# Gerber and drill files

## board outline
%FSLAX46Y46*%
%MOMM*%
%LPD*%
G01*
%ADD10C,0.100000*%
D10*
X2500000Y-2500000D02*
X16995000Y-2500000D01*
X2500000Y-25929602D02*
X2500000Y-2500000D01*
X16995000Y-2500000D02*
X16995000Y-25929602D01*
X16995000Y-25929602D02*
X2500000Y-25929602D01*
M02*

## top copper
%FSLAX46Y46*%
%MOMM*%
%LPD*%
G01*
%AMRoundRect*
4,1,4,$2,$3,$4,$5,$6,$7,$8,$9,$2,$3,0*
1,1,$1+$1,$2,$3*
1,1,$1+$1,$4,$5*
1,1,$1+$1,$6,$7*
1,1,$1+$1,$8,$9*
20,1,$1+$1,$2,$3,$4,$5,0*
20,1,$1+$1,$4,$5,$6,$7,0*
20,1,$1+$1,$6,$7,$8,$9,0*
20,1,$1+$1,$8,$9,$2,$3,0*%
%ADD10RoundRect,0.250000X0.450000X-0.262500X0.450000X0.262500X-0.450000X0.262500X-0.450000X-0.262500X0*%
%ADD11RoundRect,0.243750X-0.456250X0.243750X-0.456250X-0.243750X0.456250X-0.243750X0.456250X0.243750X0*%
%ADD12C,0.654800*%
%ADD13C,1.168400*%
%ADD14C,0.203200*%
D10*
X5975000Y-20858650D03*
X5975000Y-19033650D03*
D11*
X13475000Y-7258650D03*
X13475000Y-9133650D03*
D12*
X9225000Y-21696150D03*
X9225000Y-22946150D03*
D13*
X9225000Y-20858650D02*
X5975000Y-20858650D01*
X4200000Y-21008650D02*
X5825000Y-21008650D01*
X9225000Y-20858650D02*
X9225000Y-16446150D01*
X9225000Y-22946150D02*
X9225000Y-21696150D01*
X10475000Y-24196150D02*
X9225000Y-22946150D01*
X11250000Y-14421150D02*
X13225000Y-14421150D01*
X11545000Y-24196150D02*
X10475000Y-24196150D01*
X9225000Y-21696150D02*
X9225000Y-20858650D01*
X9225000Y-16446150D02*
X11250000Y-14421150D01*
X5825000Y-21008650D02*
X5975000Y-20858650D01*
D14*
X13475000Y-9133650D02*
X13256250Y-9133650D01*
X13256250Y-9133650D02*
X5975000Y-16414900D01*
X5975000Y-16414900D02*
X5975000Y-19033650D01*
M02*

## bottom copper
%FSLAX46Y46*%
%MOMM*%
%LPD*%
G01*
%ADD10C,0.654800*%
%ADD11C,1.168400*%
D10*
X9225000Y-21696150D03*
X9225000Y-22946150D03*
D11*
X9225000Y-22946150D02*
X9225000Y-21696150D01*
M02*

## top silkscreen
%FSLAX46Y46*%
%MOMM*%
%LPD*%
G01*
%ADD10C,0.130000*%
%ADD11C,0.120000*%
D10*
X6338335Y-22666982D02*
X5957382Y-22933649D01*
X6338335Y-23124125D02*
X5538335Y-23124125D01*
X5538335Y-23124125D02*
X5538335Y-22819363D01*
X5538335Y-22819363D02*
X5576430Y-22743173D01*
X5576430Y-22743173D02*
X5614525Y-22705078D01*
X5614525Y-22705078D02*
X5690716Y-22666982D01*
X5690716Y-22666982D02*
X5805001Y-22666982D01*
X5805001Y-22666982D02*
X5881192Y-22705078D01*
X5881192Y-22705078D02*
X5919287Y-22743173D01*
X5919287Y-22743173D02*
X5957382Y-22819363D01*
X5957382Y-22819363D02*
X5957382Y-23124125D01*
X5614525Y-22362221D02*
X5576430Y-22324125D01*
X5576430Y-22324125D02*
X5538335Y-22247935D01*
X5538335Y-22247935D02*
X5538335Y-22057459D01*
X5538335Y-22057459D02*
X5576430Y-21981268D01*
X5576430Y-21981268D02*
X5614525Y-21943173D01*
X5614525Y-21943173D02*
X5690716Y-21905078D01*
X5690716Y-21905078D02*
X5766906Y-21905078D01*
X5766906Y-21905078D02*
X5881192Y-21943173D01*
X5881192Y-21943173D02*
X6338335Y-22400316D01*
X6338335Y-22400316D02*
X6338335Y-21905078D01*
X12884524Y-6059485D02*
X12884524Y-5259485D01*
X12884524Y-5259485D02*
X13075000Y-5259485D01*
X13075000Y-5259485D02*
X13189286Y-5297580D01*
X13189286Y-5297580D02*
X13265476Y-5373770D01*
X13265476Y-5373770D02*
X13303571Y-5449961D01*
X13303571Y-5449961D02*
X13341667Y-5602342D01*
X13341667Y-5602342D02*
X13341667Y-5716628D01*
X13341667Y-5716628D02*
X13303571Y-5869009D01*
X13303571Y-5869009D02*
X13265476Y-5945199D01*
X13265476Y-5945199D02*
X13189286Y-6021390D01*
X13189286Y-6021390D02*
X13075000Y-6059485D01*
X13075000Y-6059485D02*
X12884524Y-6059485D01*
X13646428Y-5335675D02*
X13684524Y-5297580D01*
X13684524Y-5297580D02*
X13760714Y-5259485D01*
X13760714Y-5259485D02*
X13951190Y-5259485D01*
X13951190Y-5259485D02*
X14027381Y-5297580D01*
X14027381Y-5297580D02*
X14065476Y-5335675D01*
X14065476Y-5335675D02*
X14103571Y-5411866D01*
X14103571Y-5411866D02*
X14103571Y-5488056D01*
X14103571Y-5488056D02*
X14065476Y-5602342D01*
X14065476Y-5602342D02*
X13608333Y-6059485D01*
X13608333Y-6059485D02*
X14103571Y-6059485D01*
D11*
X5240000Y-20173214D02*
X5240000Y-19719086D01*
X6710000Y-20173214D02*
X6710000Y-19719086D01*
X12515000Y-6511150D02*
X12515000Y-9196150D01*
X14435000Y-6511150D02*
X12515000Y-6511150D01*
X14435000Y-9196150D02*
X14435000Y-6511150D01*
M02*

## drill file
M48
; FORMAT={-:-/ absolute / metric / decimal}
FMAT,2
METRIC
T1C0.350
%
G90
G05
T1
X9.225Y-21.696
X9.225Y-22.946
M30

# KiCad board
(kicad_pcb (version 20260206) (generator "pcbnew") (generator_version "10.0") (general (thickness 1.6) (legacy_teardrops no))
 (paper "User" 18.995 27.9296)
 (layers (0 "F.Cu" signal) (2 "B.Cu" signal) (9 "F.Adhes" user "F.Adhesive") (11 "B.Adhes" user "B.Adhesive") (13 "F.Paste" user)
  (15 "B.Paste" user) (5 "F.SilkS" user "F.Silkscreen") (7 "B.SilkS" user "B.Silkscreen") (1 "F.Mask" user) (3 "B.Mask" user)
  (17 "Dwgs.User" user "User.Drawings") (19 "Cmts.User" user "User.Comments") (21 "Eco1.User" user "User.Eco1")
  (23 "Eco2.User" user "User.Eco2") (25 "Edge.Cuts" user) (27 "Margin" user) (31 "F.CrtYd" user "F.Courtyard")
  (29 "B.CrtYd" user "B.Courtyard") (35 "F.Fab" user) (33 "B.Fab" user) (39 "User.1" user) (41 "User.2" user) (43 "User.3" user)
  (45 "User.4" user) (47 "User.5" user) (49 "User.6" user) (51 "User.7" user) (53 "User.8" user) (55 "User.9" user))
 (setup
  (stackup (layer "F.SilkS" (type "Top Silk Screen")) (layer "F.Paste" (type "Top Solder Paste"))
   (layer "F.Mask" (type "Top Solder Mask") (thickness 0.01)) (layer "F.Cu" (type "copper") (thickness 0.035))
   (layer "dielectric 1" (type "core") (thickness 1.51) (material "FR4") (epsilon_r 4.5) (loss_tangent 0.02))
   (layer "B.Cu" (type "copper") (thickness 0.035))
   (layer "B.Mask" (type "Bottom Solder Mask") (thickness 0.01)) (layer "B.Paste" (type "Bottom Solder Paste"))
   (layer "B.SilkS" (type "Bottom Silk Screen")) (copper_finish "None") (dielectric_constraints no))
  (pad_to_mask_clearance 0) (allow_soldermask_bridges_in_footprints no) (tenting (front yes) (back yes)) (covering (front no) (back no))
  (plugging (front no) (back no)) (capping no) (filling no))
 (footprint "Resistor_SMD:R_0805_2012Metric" (layer "F.Cu") (at 5.975 19.94615 90)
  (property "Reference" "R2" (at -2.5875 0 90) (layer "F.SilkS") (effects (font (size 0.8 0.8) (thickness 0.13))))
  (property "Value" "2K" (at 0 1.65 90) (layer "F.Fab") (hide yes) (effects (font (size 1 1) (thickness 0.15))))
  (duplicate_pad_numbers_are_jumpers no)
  (fp_line (start -0.227064 -0.735) (end 0.227064 -0.735) (stroke (width 0.12) (type solid)) (layer "F.SilkS"))
  (fp_line (start -0.227064 0.735) (end 0.227064 0.735) (stroke (width 0.12) (type solid)) (layer "F.SilkS"))
  (pad "1" smd roundrect (at -0.9125 0 90) (size 1.025 1.4) (layers "F.Cu" "F.Mask" "F.Paste") (roundrect_rratio 0.243902439) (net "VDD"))
  (pad "2" smd roundrect (at 0.9125 0 90) (size 1.025 1.4) (layers "F.Cu" "F.Mask" "F.Paste") (roundrect_rratio 0.243902439)
   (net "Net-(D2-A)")))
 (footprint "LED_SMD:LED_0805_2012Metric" (layer "F.Cu") (at 13.475 8.19615 -90)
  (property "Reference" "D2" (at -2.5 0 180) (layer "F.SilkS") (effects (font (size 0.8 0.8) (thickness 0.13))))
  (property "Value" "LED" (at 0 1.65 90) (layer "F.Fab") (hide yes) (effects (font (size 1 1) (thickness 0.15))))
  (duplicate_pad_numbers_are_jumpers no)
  (fp_line (start -1.685 0.96) (end 1 0.96) (stroke (width 0.12) (type solid)) (layer "F.SilkS"))
  (fp_line (start -1.685 -0.96) (end -1.685 0.96) (stroke (width 0.12) (type solid)) (layer "F.SilkS"))
  (fp_line (start 1 -0.96) (end -1.685 -0.96) (stroke (width 0.12) (type solid)) (layer "F.SilkS"))
  (pad "1" smd roundrect (at -0.9375 0 270) (size 0.975 1.4) (layers "F.Cu" "F.Mask" "F.Paste") (roundrect_rratio 0.25) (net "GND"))
  (pad "2" smd roundrect (at 0.9375 0 270) (size 0.975 1.4) (layers "F.Cu" "F.Mask" "F.Paste") (roundrect_rratio 0.25) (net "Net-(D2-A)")))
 (gr_line (start 2.5 2.5) (end 16.995 2.5) (stroke (width 0.1) (type default)) (layer "Edge.Cuts"))
 (gr_line (start 2.5 25.929602) (end 2.5 2.5) (stroke (width 0.1) (type default)) (layer "Edge.Cuts"))
 (gr_line (start 16.995 2.5) (end 16.995 25.929602) (stroke (width 0.1) (type default)) (layer "Edge.Cuts"))
 (gr_line (start 16.995 25.929602) (end 2.5 25.929602) (stroke (width 0.1) (type default)) (layer "Edge.Cuts"))
 (segment (start 9.225 20.85865) (end 5.975 20.85865) (width 1.1684) (layer "F.Cu") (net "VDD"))
 (segment (start 4.2 21.00865) (end 5.825 21.00865) (width 1.1684) (layer "F.Cu") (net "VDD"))
 (segment (start 9.225 20.85865) (end 9.225 16.44615) (width 1.1684) (layer "F.Cu") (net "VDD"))
 (segment (start 9.225 22.94615) (end 9.225 21.69615) (width 1.1684) (layer "F.Cu") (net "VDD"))
 (segment (start 10.475 24.19615) (end 9.225 22.94615) (width 1.1684) (layer "F.Cu") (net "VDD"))
 (segment (start 11.25 14.42115) (end 13.225 14.42115) (width 1.1684) (layer "F.Cu") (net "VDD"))
 (segment (start 11.545 24.19615) (end 10.475 24.19615) (width 1.1684) (layer "F.Cu") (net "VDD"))
 (segment (start 9.225 21.69615) (end 9.225 20.85865) (width 1.1684) (layer "F.Cu") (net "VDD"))
 (segment (start 9.225 16.44615) (end 11.25 14.42115) (width 1.1684) (layer "F.Cu") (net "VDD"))
 (segment (start 5.825 21.00865) (end 5.975 20.85865) (width 1.1684) (layer "F.Cu") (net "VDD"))
 (via (at 9.225 21.69615) (size 0.6548) (drill 0.35) (layers "F.Cu" "B.Cu") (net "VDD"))
 (via (at 9.225 22.94615) (size 0.6548) (drill 0.35) (layers "F.Cu" "B.Cu") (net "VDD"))
 (segment (start 9.225 22.94615) (end 9.225 21.69615) (width 1.1684) (layer "B.Cu") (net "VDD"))
 (segment (start 13.475 9.13365) (end 13.25625 9.13365) (width 0.2032) (layer "F.Cu") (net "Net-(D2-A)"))
 (segment (start 13.25625 9.13365) (end 5.975 16.4149) (width 0.2032) (layer "F.Cu") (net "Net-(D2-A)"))
 (segment (start 5.975 16.4149) (end 5.975 19.03365) (width 0.2032) (layer "F.Cu") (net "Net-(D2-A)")))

